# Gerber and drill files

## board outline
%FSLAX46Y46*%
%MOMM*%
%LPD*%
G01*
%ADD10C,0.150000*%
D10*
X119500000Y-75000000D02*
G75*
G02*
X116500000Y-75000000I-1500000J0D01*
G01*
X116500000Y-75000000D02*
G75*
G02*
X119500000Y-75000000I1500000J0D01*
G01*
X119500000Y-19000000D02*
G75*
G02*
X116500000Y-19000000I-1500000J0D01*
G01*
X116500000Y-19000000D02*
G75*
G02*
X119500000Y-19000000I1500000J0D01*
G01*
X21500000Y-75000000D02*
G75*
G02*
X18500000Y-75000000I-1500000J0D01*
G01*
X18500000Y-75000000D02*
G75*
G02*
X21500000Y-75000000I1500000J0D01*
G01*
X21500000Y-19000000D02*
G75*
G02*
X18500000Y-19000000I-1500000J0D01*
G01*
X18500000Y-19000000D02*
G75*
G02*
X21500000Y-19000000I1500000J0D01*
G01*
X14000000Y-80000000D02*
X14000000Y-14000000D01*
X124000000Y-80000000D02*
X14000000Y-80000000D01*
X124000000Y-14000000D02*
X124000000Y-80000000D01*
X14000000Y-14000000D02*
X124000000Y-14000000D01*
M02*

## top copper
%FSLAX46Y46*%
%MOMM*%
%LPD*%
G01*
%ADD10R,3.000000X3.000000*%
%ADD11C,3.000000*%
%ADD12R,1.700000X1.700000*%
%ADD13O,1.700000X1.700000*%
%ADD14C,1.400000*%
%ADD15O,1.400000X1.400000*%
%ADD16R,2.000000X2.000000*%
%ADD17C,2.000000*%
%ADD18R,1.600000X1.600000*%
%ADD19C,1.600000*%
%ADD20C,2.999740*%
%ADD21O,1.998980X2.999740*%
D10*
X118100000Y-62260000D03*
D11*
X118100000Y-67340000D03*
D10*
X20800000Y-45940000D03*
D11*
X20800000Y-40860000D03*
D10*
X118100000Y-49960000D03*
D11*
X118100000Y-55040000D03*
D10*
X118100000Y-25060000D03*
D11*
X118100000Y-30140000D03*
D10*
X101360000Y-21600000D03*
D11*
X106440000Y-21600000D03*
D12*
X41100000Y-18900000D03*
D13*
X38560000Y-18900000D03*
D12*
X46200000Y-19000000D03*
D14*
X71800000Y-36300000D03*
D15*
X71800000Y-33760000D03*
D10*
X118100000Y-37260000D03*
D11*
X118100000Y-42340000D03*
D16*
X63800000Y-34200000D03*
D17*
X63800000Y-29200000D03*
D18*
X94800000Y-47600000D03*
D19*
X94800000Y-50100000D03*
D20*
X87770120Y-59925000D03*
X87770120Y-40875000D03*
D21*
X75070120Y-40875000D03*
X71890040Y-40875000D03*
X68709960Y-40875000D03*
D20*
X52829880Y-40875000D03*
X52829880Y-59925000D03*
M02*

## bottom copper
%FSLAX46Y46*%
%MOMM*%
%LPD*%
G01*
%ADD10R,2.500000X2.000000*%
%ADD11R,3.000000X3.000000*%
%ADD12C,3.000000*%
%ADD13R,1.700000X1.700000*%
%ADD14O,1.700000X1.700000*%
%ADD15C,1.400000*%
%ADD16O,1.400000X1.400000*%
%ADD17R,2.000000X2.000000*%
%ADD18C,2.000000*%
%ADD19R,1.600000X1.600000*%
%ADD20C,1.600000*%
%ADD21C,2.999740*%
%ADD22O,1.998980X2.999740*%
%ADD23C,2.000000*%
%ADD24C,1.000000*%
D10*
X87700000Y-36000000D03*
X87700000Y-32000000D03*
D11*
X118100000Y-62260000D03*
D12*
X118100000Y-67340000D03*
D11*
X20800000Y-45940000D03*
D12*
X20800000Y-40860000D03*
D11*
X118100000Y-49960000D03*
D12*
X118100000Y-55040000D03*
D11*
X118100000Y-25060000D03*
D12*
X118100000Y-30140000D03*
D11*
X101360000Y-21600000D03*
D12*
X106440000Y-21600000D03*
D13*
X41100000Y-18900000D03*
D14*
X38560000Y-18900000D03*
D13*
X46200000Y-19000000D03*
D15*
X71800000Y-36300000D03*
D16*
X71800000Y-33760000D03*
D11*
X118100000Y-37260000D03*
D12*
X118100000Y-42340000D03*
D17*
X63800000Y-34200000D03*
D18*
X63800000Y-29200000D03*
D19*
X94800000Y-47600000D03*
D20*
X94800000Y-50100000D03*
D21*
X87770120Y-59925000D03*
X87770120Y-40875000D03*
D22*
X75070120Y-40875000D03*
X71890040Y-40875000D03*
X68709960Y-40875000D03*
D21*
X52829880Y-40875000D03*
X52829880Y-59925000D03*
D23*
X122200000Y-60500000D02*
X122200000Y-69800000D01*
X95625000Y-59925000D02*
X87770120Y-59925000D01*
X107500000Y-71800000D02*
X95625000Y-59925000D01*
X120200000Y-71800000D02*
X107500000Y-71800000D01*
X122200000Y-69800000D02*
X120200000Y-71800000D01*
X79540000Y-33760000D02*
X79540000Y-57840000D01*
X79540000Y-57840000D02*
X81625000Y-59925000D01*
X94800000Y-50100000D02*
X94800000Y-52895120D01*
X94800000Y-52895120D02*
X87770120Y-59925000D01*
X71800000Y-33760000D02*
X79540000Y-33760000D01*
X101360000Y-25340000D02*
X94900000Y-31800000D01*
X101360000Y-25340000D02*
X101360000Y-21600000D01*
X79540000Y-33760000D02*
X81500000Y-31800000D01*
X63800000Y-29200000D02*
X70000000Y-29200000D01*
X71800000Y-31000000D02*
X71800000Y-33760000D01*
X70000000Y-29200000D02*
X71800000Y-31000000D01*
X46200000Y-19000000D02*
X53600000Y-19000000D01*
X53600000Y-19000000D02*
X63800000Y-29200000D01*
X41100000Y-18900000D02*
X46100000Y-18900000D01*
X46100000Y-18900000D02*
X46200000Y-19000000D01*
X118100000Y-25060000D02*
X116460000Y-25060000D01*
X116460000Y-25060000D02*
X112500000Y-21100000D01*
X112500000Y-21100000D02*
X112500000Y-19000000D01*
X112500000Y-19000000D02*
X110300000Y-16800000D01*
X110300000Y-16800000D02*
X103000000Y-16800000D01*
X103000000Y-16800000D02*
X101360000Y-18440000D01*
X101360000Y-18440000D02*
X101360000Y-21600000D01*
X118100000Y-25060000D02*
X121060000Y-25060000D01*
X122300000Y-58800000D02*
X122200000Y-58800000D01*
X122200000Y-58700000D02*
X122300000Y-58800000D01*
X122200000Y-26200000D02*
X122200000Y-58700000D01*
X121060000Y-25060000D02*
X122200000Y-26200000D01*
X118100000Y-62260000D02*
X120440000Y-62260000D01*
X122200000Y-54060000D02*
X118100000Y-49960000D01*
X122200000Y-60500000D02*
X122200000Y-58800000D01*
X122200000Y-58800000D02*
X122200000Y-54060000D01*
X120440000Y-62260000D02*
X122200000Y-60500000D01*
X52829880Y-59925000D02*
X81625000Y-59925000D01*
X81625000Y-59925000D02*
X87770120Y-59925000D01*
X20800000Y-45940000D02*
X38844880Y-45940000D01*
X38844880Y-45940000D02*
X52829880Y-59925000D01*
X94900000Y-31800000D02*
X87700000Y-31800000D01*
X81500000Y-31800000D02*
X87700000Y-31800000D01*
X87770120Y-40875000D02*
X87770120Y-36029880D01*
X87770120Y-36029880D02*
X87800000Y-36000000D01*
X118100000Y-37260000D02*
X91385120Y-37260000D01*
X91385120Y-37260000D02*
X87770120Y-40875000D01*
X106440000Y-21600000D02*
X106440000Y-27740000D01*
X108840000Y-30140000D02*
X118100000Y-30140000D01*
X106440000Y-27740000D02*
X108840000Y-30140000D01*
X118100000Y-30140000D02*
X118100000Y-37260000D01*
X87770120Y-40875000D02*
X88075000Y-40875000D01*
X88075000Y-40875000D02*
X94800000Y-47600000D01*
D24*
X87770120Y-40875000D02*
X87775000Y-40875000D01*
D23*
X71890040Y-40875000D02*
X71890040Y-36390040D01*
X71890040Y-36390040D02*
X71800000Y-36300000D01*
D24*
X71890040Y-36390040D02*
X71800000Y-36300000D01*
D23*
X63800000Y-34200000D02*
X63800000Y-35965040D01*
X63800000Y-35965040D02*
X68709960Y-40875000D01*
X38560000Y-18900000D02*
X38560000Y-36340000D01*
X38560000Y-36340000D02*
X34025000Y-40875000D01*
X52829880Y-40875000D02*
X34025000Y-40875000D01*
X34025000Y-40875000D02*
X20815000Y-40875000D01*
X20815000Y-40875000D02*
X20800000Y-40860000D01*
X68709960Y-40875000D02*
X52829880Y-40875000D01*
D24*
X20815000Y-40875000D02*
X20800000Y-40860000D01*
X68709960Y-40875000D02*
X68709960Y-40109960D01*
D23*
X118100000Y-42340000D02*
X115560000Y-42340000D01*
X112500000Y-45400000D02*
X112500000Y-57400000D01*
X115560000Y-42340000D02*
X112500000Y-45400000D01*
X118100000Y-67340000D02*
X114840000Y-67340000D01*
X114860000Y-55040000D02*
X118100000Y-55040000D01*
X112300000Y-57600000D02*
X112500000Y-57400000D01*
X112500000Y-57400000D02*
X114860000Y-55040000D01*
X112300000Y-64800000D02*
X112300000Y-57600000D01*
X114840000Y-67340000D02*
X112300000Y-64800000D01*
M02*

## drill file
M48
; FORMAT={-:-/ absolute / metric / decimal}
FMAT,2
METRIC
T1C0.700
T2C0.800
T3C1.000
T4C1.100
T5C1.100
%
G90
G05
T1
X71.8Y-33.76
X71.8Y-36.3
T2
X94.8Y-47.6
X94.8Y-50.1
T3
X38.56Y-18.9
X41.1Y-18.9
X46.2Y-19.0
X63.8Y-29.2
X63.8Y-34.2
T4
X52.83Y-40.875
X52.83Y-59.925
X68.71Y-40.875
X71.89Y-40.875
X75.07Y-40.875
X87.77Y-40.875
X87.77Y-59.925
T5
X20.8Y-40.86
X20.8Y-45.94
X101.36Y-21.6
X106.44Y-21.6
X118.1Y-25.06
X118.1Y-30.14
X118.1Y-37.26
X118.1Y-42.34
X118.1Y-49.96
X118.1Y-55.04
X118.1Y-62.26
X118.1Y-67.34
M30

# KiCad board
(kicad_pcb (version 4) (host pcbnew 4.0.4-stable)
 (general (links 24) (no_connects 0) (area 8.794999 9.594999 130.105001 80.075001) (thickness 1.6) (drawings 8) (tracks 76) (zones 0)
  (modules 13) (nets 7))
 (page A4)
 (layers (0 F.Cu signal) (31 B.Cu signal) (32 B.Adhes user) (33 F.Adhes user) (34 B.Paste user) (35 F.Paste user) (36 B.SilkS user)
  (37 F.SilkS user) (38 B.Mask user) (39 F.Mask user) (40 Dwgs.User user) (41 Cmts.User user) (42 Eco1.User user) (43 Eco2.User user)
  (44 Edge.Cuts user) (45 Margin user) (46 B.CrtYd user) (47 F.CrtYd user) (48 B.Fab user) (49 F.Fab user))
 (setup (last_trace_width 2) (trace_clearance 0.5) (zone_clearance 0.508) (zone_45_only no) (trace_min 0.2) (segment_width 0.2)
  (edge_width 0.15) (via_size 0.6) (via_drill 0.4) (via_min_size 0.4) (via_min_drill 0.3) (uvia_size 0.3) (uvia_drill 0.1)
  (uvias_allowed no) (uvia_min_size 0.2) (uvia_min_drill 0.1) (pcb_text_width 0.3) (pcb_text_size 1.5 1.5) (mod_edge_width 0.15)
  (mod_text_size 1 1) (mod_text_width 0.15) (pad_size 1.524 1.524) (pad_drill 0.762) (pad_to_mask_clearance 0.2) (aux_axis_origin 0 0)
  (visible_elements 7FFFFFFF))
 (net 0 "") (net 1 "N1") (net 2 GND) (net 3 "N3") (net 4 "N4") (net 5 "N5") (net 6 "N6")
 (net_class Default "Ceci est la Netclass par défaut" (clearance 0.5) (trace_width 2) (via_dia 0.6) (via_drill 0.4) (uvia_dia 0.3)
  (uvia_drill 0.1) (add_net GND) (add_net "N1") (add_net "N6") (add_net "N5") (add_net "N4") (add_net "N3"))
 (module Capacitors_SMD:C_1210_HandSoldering (layer B.Cu) (at 87.7 34 90)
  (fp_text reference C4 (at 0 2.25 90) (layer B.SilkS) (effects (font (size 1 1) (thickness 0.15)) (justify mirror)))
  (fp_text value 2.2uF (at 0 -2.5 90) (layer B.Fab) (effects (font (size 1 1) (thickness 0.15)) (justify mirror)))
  (pad 1 smd rect (at -2 0 90) (size 2 2.5) (layers B.Cu B.Paste B.Mask) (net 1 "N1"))
  (pad 2 smd rect (at 2 0 90) (size 2 2.5) (layers B.Cu B.Paste B.Mask) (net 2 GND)))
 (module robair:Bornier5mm (layer F.Cu) (at 118.1 64.8 270)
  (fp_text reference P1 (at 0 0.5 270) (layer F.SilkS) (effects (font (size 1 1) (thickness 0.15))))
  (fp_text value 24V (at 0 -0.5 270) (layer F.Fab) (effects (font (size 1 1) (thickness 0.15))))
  (pad 1 thru_hole rect (at -2.54 0 270) (size 3 3) (drill 1.1) (layers *.Cu *.Mask) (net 2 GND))
  (pad 2 thru_hole circle (at 2.54 0 270) (size 3 3) (drill 1.1) (layers *.Cu *.Mask) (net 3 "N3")))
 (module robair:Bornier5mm (layer F.Cu) (at 20.8 43.4 90)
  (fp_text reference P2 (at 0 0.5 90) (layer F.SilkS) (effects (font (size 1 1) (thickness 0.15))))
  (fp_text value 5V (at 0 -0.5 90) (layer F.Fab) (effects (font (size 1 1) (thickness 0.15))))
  (pad 1 thru_hole rect (at -2.54 0 90) (size 3 3) (drill 1.1) (layers *.Cu *.Mask) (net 2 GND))
  (pad 2 thru_hole circle (at 2.54 0 90) (size 3 3) (drill 1.1) (layers *.Cu *.Mask) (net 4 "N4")))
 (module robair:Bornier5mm (layer F.Cu) (at 118.1 52.5 270)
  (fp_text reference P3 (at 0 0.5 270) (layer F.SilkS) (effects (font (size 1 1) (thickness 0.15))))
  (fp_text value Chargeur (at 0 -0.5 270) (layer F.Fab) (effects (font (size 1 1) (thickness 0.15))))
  (pad 1 thru_hole rect (at -2.54 0 270) (size 3 3) (drill 1.1) (layers *.Cu *.Mask) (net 2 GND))
  (pad 2 thru_hole circle (at 2.54 0 270) (size 3 3) (drill 1.1) (layers *.Cu *.Mask) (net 3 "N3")))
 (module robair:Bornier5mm (layer F.Cu) (at 118.1 27.6 270)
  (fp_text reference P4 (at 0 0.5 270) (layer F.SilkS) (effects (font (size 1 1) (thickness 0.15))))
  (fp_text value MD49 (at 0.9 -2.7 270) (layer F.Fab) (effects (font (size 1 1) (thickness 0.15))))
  (pad 1 thru_hole rect (at -2.54 0 270) (size 3 3) (drill 1.1) (layers *.Cu *.Mask) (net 2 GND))
  (pad 2 thru_hole circle (at 2.54 0 270) (size 3 3) (drill 1.1) (layers *.Cu *.Mask) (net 1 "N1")))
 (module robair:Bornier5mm (layer F.Cu) (at 103.9 21.6)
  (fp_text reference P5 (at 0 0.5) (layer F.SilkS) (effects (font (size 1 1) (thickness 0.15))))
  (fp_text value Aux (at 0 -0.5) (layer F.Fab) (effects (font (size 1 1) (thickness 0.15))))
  (pad 1 thru_hole rect (at -2.54 0) (size 3 3) (drill 1.1) (layers *.Cu *.Mask) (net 2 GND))
  (pad 2 thru_hole circle (at 2.54 0) (size 3 3) (drill 1.1) (layers *.Cu *.Mask) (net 1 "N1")))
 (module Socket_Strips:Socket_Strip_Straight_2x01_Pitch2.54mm (layer F.Cu) (at 41.1 18.9)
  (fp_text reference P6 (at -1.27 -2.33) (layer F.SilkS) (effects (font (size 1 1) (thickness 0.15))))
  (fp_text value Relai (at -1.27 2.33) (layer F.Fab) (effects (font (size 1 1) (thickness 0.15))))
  (pad 1 thru_hole rect (at 0 0) (size 1.7 1.7) (drill 1) (layers *.Cu *.Mask) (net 2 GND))
  (pad 2 thru_hole oval (at -2.54 0) (size 1.7 1.7) (drill 1) (layers *.Cu *.Mask) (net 4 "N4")))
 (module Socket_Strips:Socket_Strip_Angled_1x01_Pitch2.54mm (layer F.Cu) (at 46.2 19 90)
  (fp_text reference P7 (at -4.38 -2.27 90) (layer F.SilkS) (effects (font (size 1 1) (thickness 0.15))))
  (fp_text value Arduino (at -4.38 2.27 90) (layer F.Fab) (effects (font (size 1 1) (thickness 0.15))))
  (pad 1 thru_hole rect (at 0 0 90) (size 1.7 1.7) (drill 1) (layers *.Cu *.Mask) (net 2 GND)))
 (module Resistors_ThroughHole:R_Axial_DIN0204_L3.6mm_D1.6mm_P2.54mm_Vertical (layer F.Cu) (at 71.8 36.3 90)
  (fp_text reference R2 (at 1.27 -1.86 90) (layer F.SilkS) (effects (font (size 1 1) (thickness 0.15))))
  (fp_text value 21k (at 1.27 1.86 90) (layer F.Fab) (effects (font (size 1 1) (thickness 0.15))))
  (pad 1 thru_hole circle (at 0 0 90) (size 1.4 1.4) (drill 0.7) (layers *.Cu *.Mask) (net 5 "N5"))
  (pad 2 thru_hole oval (at 2.54 0 90) (size 1.4 1.4) (drill 0.7) (layers *.Cu *.Mask) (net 2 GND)))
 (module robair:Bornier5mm (layer F.Cu) (at 118.1 39.8 270)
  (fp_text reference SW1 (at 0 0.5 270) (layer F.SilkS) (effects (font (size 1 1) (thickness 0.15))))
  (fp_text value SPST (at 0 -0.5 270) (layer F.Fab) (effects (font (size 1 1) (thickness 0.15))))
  (pad 1 thru_hole rect (at -2.54 0 270) (size 3 3) (drill 1.1) (layers *.Cu *.Mask) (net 1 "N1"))
  (pad 2 thru_hole circle (at 2.54 0 270) (size 3 3) (drill 1.1) (layers *.Cu *.Mask) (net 3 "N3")))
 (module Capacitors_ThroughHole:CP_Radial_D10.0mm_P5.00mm (layer F.Cu) (at 63.8 34.2 90)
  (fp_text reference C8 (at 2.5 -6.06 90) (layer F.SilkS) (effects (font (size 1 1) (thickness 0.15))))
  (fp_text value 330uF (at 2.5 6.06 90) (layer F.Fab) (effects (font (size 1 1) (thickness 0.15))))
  (pad 1 thru_hole rect (at 0 0 90) (size 2 2) (drill 1) (layers *.Cu *.Mask) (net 4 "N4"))
  (pad 2 thru_hole circle (at 5 0 90) (size 2 2) (drill 1) (layers *.Cu *.Mask) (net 2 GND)))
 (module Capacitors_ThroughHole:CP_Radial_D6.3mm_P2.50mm (layer F.Cu) (at 94.8 47.6 270)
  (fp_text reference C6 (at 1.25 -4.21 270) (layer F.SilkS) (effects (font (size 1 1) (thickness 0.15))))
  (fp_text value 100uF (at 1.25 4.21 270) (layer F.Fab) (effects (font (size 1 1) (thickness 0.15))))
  (pad 1 thru_hole rect (at 0 0 270) (size 1.6 1.6) (drill 0.8) (layers *.Cu *.Mask) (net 1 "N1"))
  (pad 2 thru_hole circle (at 2.5 0 270) (size 1.6 1.6) (drill 0.8) (layers *.Cu *.Mask) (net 2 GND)))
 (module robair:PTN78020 (layer F.Cu) (at 70.3 50.4 180)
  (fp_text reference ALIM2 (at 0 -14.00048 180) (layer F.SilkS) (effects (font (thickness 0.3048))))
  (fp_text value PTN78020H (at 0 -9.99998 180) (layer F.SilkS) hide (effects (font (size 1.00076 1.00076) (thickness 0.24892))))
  (pad 1 thru_hole circle (at -17.47012 -9.525 180) (size 2.99974 2.99974) (drill 1.09982) (layers *.Cu *.Mask) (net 2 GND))
  (pad 2 thru_hole circle (at -17.47012 9.525 180) (size 2.99974 2.99974) (drill 1.09982) (layers *.Cu *.Mask) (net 1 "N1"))
  (pad 3 thru_hole oval (at -4.77012 9.525 180) (size 1.99898 2.99974) (drill 1.09982) (layers *.Cu *.Mask) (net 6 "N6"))
  (pad 4 thru_hole oval (at -1.59004 9.525 180) (size 1.99898 2.99974) (drill 1.09982) (layers *.Cu *.Mask) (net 5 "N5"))
  (pad 5 thru_hole oval (at 1.59004 9.525 180) (size 1.99898 2.99974) (drill 1.09982) (layers *.Cu *.Mask) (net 4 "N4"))
  (pad 6 thru_hole circle (at 17.47012 9.525 180) (size 2.99974 2.99974) (drill 1.09982) (layers *.Cu *.Mask) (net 4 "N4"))
  (pad 7 thru_hole circle (at 17.47012 -9.525 180) (size 2.99974 2.99974) (drill 1.09982) (layers *.Cu *.Mask) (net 2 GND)))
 (gr_circle (center 118 75) (end 119.5 75) (layer Edge.Cuts) (width 0.15))
 (gr_circle (center 118 19) (end 119.5 19) (layer Edge.Cuts) (width 0.15))
 (gr_circle (center 20 75) (end 18.5 75) (layer Edge.Cuts) (width 0.15))
 (gr_circle (center 20 19) (end 18.5 19) (layer Edge.Cuts) (width 0.15))
 (gr_line (start 14 80) (end 14 14) (angle 90) (layer Edge.Cuts) (width 0.15))
 (gr_line (start 124 80) (end 14 80) (angle 90) (layer Edge.Cuts) (width 0.15))
 (gr_line (start 124 14) (end 124 80) (angle 90) (layer Edge.Cuts) (width 0.15))
 (gr_line (start 14 14) (end 124 14) (angle 90) (layer Edge.Cuts) (width 0.15))
 (segment (start 122.2 60.5) (end 122.2 69.8) (width 2) (layer B.Cu) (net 2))
 (segment (start 95.625 59.925) (end 87.77012 59.925) (width 2) (layer B.Cu) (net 2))
 (segment (start 107.5 71.8) (end 95.625 59.925) (width 2) (layer B.Cu) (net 2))
 (segment (start 120.2 71.8) (end 107.5 71.8) (width 2) (layer B.Cu) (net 2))
 (segment (start 122.2 69.8) (end 120.2 71.8) (width 2) (layer B.Cu) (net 2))
 (segment (start 79.54 33.76) (end 79.54 57.84) (width 2) (layer B.Cu) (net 2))
 (segment (start 79.54 57.84) (end 81.625 59.925) (width 2) (layer B.Cu) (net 2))
 (segment (start 94.8 50.1) (end 94.8 52.89512) (width 2) (layer B.Cu) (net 2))
 (segment (start 94.8 52.89512) (end 87.77012 59.925) (width 2) (layer B.Cu) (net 2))
 (segment (start 71.8 33.76) (end 79.54 33.76) (width 2) (layer B.Cu) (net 2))
 (segment (start 101.36 25.34) (end 94.9 31.8) (width 2) (layer B.Cu) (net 2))
 (segment (start 101.36 25.34) (end 101.36 21.6) (width 2) (layer B.Cu) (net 2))
 (segment (start 79.54 33.76) (end 81.5 31.8) (width 2) (layer B.Cu) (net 2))
 (segment (start 63.8 29.2) (end 70 29.2) (width 2) (layer B.Cu) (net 2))
 (segment (start 71.8 31) (end 71.8 33.76) (width 2) (layer B.Cu) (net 2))
 (segment (start 70 29.2) (end 71.8 31) (width 2) (layer B.Cu) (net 2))
 (segment (start 46.2 19) (end 53.6 19) (width 2) (layer B.Cu) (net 2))
 (segment (start 53.6 19) (end 63.8 29.2) (width 2) (layer B.Cu) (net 2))
 (segment (start 41.1 18.9) (end 46.1 18.9) (width 2) (layer B.Cu) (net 2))
 (segment (start 46.1 18.9) (end 46.2 19) (width 2) (layer B.Cu) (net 2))
 (segment (start 118.1 25.06) (end 116.46 25.06) (width 2) (layer B.Cu) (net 2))
 (segment (start 116.46 25.06) (end 112.5 21.1) (width 2) (layer B.Cu) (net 2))
 (segment (start 112.5 21.1) (end 112.5 19) (width 2) (layer B.Cu) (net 2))
 (segment (start 112.5 19) (end 110.3 16.8) (width 2) (layer B.Cu) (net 2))
 (segment (start 110.3 16.8) (end 103 16.8) (width 2) (layer B.Cu) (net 2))
 (segment (start 103 16.8) (end 101.36 18.44) (width 2) (layer B.Cu) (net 2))
 (segment (start 101.36 18.44) (end 101.36 21.6) (width 2) (layer B.Cu) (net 2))
 (segment (start 118.1 25.06) (end 121.06 25.06) (width 2) (layer B.Cu) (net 2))
 (segment (start 122.3 58.8) (end 122.2 58.8) (width 2) (layer B.Cu) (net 2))
 (segment (start 122.2 58.7) (end 122.3 58.8) (width 2) (layer B.Cu) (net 2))
 (segment (start 122.2 26.2) (end 122.2 58.7) (width 2) (layer B.Cu) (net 2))
 (segment (start 121.06 25.06) (end 122.2 26.2) (width 2) (layer B.Cu) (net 2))
 (segment (start 118.1 62.26) (end 120.44 62.26) (width 2) (layer B.Cu) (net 2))
 (segment (start 122.2 54.06) (end 118.1 49.96) (width 2) (layer B.Cu) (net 2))
 (segment (start 122.2 60.5) (end 122.2 58.8) (width 2) (layer B.Cu) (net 2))
 (segment (start 122.2 58.8) (end 122.2 54.06) (width 2) (layer B.Cu) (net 2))
 (segment (start 120.44 62.26) (end 122.2 60.5) (width 2) (layer B.Cu) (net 2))
 (segment (start 52.82988 59.925) (end 81.625 59.925) (width 2) (layer B.Cu) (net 2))
 (segment (start 81.625 59.925) (end 87.77012 59.925) (width 2) (layer B.Cu) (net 2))
 (segment (start 20.8 45.94) (end 38.84488 45.94) (width 2) (layer B.Cu) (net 2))
 (segment (start 38.84488 45.94) (end 52.82988 59.925) (width 2) (layer B.Cu) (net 2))
 (segment (start 94.9 31.8) (end 87.7 31.8) (width 2) (layer B.Cu) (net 2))
 (segment (start 81.5 31.8) (end 87.7 31.8) (width 2) (layer B.Cu) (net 2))
 (segment (start 87.77012 40.875) (end 87.77012 36.02988) (width 2) (layer B.Cu) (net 1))
 (segment (start 87.77012 36.02988) (end 87.8 36) (width 2) (layer B.Cu) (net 1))
 (segment (start 118.1 37.26) (end 91.38512 37.26) (width 2) (layer B.Cu) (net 1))
 (segment (start 91.38512 37.26) (end 87.77012 40.875) (width 2) (layer B.Cu) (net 1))
 (segment (start 106.44 21.6) (end 106.44 27.74) (width 2) (layer B.Cu) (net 1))
 (segment (start 108.84 30.14) (end 118.1 30.14) (width 2) (layer B.Cu) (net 1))
 (segment (start 106.44 27.74) (end 108.84 30.14) (width 2) (layer B.Cu) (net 1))
 (segment (start 118.1 30.14) (end 118.1 37.26) (width 2) (layer B.Cu) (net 1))
 (segment (start 87.77012 40.875) (end 88.075 40.875) (width 2) (layer B.Cu) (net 1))
 (segment (start 88.075 40.875) (end 94.8 47.6) (width 2) (layer B.Cu) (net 1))
 (segment (start 87.77012 40.875) (end 87.775 40.875) (width 1) (layer B.Cu) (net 1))
 (segment (start 71.89004 40.875) (end 71.89004 36.39004) (width 2) (layer B.Cu) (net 5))
 (segment (start 71.89004 36.39004) (end 71.8 36.3) (width 2) (layer B.Cu) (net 5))
 (segment (start 71.89004 36.39004) (end 71.8 36.3) (width 1) (layer B.Cu) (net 5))
 (segment (start 63.8 34.2) (end 63.8 35.96504) (width 2) (layer B.Cu) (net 4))
 (segment (start 63.8 35.96504) (end 68.70996 40.875) (width 2) (layer B.Cu) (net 4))
 (segment (start 38.56 18.9) (end 38.56 36.34) (width 2) (layer B.Cu) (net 4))
 (segment (start 38.56 36.34) (end 34.025 40.875) (width 2) (layer B.Cu) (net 4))
 (segment (start 52.82988 40.875) (end 34.025 40.875) (width 2) (layer B.Cu) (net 4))
 (segment (start 34.025 40.875) (end 20.815 40.875) (width 2) (layer B.Cu) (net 4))
 (segment (start 20.815 40.875) (end 20.8 40.86) (width 2) (layer B.Cu) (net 4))
 (segment (start 68.70996 40.875) (end 52.82988 40.875) (width 2) (layer B.Cu) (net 4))
 (segment (start 20.815 40.875) (end 20.8 40.86) (width 1) (layer B.Cu) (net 4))
 (segment (start 68.70996 40.875) (end 68.70996 40.10996) (width 1) (layer B.Cu) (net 4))
 (segment (start 118.1 42.34) (end 115.56 42.34) (width 2) (layer B.Cu) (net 3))
 (segment (start 112.5 45.4) (end 112.5 57.4) (width 2) (layer B.Cu) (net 3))
 (segment (start 115.56 42.34) (end 112.5 45.4) (width 2) (layer B.Cu) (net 3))
 (segment (start 118.1 67.34) (end 114.84 67.34) (width 2) (layer B.Cu) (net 3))
 (segment (start 114.86 55.04) (end 118.1 55.04) (width 2) (layer B.Cu) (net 3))
 (segment (start 112.3 57.6) (end 112.5 57.4) (width 2) (layer B.Cu) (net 3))
 (segment (start 112.5 57.4) (end 114.86 55.04) (width 2) (layer B.Cu) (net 3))
 (segment (start 112.3 64.8) (end 112.3 57.6) (width 2) (layer B.Cu) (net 3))
 (segment (start 114.84 67.34) (end 112.3 64.8) (width 2) (layer B.Cu) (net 3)))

